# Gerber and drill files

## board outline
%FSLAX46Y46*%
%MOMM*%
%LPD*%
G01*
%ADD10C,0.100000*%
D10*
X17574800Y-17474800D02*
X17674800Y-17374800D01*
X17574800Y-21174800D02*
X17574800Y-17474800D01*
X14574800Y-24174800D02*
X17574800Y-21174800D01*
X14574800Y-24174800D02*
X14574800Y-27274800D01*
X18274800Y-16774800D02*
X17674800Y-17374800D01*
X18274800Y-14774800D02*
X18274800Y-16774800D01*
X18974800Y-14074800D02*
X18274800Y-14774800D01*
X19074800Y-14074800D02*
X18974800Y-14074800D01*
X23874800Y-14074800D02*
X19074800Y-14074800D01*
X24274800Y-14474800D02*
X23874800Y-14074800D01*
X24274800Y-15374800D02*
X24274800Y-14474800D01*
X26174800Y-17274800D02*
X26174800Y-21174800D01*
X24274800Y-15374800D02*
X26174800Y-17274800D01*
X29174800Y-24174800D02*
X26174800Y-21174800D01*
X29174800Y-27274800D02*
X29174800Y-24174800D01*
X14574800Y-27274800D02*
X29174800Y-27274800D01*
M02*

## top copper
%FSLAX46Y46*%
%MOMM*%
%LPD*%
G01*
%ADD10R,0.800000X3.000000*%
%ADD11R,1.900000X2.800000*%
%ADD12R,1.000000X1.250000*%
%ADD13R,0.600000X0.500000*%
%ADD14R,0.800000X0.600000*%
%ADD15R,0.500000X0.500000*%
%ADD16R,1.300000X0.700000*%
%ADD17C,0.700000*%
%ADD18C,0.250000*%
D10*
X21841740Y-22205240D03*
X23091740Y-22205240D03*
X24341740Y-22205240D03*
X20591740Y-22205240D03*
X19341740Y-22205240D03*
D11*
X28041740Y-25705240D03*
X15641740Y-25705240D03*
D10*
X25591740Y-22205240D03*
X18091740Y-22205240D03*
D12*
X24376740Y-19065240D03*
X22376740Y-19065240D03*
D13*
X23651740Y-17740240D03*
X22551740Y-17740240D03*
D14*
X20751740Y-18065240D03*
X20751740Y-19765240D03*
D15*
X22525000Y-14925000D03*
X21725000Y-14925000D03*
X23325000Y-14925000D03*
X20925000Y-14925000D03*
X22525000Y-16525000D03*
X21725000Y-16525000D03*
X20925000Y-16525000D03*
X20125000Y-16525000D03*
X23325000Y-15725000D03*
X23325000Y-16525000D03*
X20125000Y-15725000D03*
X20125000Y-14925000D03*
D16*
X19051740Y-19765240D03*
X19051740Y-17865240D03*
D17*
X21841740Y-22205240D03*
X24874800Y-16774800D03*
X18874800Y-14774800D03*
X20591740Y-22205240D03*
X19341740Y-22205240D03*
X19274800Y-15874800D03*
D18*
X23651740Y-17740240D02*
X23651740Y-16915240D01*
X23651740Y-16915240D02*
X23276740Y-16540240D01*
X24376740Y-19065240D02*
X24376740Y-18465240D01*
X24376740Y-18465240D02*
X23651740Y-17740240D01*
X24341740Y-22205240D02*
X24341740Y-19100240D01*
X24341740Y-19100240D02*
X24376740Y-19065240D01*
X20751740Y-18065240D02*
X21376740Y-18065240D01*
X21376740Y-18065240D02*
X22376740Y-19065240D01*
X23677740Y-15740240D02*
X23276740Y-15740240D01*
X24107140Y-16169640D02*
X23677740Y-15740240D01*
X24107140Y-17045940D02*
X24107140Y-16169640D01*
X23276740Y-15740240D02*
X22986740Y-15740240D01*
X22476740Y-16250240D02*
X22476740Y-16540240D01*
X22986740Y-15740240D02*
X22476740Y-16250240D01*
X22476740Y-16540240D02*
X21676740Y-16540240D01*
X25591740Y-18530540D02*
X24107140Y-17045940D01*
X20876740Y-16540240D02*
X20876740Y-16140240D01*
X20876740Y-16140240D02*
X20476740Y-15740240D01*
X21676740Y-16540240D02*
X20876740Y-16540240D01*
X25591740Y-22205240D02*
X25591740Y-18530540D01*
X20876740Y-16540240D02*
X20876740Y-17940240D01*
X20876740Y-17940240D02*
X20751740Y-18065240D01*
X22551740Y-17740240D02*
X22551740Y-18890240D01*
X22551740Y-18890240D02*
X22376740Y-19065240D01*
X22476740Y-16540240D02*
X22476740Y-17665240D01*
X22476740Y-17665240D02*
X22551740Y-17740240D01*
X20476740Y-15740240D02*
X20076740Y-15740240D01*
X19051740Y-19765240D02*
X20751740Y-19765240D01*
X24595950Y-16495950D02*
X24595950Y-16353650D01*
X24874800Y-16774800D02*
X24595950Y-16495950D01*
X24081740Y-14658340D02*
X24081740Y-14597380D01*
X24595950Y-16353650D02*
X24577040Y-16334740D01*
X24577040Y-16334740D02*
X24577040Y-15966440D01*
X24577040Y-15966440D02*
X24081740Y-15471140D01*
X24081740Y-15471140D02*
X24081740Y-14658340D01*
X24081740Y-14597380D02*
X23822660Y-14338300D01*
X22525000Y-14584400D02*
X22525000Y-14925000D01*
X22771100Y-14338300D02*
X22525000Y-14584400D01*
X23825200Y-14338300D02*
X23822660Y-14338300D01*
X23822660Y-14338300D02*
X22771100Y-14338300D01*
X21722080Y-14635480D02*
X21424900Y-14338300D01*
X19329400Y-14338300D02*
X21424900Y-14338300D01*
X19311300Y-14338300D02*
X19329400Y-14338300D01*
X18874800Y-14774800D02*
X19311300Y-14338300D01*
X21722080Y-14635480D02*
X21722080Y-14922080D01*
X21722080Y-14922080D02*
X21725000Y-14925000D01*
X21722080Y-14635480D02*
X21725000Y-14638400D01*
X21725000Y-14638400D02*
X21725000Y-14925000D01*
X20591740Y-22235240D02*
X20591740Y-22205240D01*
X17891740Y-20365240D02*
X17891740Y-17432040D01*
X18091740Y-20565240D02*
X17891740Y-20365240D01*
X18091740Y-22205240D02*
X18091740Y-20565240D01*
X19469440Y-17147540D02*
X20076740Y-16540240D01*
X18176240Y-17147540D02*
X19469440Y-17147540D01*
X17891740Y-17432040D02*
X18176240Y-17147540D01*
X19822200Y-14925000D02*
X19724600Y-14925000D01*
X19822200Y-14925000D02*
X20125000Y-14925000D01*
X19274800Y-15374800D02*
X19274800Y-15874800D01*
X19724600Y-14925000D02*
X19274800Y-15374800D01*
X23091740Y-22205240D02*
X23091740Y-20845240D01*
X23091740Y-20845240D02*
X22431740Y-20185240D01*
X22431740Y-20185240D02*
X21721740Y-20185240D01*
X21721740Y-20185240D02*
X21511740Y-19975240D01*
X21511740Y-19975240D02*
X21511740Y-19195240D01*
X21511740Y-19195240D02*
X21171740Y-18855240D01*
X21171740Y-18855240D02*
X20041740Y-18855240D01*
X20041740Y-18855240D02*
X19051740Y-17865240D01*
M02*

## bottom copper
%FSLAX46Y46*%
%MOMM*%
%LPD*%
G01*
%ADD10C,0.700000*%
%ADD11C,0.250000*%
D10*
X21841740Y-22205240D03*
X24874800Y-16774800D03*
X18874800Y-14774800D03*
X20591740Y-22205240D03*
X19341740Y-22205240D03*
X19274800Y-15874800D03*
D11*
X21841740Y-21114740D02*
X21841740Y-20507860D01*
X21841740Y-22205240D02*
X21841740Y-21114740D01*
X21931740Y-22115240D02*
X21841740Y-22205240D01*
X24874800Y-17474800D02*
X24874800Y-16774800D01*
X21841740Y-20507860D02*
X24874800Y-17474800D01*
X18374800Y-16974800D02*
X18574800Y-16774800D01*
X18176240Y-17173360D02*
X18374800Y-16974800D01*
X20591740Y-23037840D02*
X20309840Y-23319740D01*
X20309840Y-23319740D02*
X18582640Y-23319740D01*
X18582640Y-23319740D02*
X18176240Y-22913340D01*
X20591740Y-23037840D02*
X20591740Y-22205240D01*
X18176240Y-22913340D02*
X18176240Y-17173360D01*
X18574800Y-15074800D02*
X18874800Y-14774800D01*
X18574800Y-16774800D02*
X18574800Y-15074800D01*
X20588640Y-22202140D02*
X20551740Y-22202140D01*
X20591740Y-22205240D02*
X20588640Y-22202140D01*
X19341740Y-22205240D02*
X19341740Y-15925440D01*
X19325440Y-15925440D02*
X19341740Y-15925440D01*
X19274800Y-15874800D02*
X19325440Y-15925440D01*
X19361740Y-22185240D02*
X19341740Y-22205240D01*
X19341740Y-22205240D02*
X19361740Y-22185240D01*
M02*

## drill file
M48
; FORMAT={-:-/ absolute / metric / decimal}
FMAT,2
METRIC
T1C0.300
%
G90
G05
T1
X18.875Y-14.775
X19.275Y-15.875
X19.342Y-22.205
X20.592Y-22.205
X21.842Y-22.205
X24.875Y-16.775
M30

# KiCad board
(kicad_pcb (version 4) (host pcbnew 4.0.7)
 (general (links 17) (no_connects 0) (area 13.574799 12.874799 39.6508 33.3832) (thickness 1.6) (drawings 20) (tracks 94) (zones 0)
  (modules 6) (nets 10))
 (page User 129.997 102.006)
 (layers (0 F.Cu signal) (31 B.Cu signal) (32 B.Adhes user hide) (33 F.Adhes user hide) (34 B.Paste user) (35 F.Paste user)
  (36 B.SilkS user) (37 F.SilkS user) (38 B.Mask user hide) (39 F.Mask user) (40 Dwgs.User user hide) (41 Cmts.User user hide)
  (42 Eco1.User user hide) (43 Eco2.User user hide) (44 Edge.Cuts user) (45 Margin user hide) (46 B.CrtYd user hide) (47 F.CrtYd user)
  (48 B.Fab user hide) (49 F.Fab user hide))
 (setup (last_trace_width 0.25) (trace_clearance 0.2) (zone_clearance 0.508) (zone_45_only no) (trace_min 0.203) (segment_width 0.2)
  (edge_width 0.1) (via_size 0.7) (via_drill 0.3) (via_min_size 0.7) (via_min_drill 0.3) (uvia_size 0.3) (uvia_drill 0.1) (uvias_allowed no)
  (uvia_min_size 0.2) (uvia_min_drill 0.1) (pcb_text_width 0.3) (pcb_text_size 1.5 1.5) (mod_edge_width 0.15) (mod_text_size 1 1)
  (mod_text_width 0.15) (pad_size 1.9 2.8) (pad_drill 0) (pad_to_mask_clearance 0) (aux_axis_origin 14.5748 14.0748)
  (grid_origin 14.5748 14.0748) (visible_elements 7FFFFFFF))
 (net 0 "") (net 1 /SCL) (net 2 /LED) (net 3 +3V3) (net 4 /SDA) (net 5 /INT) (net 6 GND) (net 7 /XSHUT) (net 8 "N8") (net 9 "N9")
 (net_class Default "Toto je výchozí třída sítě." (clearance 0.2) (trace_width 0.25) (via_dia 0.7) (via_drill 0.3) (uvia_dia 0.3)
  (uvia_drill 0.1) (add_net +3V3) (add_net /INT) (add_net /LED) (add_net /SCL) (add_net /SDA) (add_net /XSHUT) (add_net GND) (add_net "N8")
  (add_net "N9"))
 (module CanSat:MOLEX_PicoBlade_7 (layer F.Cu) (at 21.84174 24.74524)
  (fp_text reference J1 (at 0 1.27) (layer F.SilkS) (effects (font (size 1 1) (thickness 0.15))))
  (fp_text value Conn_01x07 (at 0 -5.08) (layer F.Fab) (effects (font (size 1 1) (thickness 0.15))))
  (pad 4 smd rect (at 0 -2.54) (size 0.8 3) (layers F.Cu F.Paste F.Mask) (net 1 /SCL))
  (pad 5 smd rect (at 1.25 -2.54) (size 0.8 3) (layers F.Cu F.Paste F.Mask) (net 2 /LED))
  (pad 6 smd rect (at 2.5 -2.54) (size 0.8 3) (layers F.Cu F.Paste F.Mask) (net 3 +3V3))
  (pad 3 smd rect (at -1.25 -2.54) (size 0.8 3) (layers F.Cu F.Paste F.Mask) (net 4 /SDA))
  (pad 2 smd rect (at -2.5 -2.54) (size 0.8 3) (layers F.Cu F.Paste F.Mask) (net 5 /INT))
  (pad "" smd rect (at 6.2 0.96) (size 1.9 2.8) (layers F.Cu F.Paste F.Mask))
  (pad "" smd rect (at -6.2 0.96) (size 1.9 2.8) (layers F.Cu F.Paste F.Mask))
  (pad 7 smd rect (at 3.75 -2.54) (size 0.8 3) (layers F.Cu F.Paste F.Mask) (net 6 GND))
  (pad 1 smd rect (at -3.75 -2.54) (size 0.8 3) (layers F.Cu F.Paste F.Mask) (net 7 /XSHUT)))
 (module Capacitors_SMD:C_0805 (layer F.Cu) (at 23.37674 19.06524 180)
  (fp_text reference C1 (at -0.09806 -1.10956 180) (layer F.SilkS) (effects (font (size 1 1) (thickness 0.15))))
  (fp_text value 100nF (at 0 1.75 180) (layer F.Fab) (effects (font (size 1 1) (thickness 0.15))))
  (pad 1 smd rect (at -1 0 180) (size 1 1.25) (layers F.Cu F.Paste F.Mask) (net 3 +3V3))
  (pad 2 smd rect (at 1 0 180) (size 1 1.25) (layers F.Cu F.Paste F.Mask) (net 6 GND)))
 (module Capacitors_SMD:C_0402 (layer F.Cu) (at 23.10174 17.74024 180)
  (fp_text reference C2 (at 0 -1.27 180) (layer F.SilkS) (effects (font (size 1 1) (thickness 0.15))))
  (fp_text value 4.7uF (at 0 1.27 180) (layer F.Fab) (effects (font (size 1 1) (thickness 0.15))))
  (pad 1 smd rect (at -0.55 0 180) (size 0.6 0.5) (layers F.Cu F.Paste F.Mask) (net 3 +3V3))
  (pad 2 smd rect (at 0.55 0 180) (size 0.6 0.5) (layers F.Cu F.Paste F.Mask) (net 6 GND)))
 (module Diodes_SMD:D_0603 (layer F.Cu) (at 20.75174 18.91524 270)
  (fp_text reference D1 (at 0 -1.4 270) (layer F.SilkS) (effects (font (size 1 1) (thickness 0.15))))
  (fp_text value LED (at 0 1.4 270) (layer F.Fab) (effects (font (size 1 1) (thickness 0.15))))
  (pad 1 smd rect (at -0.85 0 270) (size 0.6 0.8) (layers F.Cu F.Paste F.Mask) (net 6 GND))
  (pad 2 smd rect (at 0.85 0 270) (size 0.6 0.8) (layers F.Cu F.Paste F.Mask) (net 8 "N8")))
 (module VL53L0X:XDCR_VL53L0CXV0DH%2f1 (layer F.Cu) (at 21.725 15.725 270)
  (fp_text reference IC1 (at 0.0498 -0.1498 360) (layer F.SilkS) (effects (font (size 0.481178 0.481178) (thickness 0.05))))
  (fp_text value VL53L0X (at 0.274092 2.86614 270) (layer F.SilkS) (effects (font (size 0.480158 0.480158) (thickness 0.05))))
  (pad 10 smd rect (at -0.8 -0.8 270) (size 0.5 0.5) (layers F.Cu F.Paste F.Mask) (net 1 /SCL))
  (pad 9 smd rect (at -0.8 0 270) (size 0.5 0.5) (layers F.Cu F.Paste F.Mask) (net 4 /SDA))
  (pad 11 smd rect (at -0.8 -1.6 270) (size 0.5 0.5) (layers F.Cu F.Paste F.Mask))
  (pad 8 smd rect (at -0.8 0.8 270) (size 0.5 0.5) (layers F.Cu F.Paste F.Mask) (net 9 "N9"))
  (pad 2 smd rect (at 0.8 -0.8 270) (size 0.5 0.5) (layers F.Cu F.Paste F.Mask) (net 6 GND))
  (pad 3 smd rect (at 0.8 0 270) (size 0.5 0.5) (layers F.Cu F.Paste F.Mask) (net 6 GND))
  (pad 4 smd rect (at 0.8 0.8 270) (size 0.5 0.5) (layers F.Cu F.Paste F.Mask) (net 6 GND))
  (pad 5 smd rect (at 0.8 1.6 270) (size 0.5 0.5) (layers F.Cu F.Paste F.Mask) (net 7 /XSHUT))
  (pad 12 smd rect (at 0 -1.6 270) (size 0.5 0.5) (layers F.Cu F.Paste F.Mask) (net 6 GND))
  (pad 1 smd rect (at 0.8 -1.6 270) (size 0.5 0.5) (layers F.Cu F.Paste F.Mask) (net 3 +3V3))
  (pad 6 smd rect (at 0 1.6 270) (size 0.5 0.5) (layers F.Cu F.Paste F.Mask) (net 6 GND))
  (pad 7 smd rect (at -0.8 1.6 270) (size 0.5 0.5) (layers F.Cu F.Paste F.Mask) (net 5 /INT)))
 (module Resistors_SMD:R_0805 (layer F.Cu) (at 19.05174 18.81524 90)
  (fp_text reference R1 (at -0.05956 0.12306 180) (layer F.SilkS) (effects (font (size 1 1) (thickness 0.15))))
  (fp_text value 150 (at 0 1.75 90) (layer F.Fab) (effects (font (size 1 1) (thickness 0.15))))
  (pad 1 smd rect (at -0.95 0 90) (size 0.7 1.3) (layers F.Cu F.Paste F.Mask) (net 8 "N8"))
  (pad 2 smd rect (at 0.95 0 90) (size 0.7 1.3) (layers F.Cu F.Paste F.Mask) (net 2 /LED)))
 (gr_line (start 17.5748 17.4748) (end 17.6748 17.3748) (angle 90) (layer Edge.Cuts) (width 0.1))
 (gr_line (start 17.5748 21.1748) (end 17.5748 17.4748) (angle 90) (layer Edge.Cuts) (width 0.1))
 (gr_line (start 14.5748 24.1748) (end 17.5748 21.1748) (angle 90) (layer Edge.Cuts) (width 0.1))
 (gr_line (start 14.5748 24.1748) (end 14.5748 27.2748) (angle 90) (layer Edge.Cuts) (width 0.1))
 (gr_line (start 18.2748 16.7748) (end 17.6748 17.3748) (angle 90) (layer Edge.Cuts) (width 0.1))
 (gr_line (start 18.2748 14.7748) (end 18.2748 16.7748) (angle 90) (layer Edge.Cuts) (width 0.1))
 (gr_line (start 18.9748 14.0748) (end 18.2748 14.7748) (angle 90) (layer Edge.Cuts) (width 0.1))
 (gr_line (start 19.0748 14.0748) (end 18.9748 14.0748) (angle 90) (layer Edge.Cuts) (width 0.1))
 (gr_line (start 23.8748 14.0748) (end 19.0748 14.0748) (angle 90) (layer Edge.Cuts) (width 0.1))
 (gr_line (start 24.2748 14.4748) (end 23.8748 14.0748) (angle 90) (layer Edge.Cuts) (width 0.1))
 (gr_line (start 24.2748 15.3748) (end 24.2748 14.4748) (angle 90) (layer Edge.Cuts) (width 0.1))
 (gr_line (start 26.1748 17.2748) (end 26.1748 21.1748) (angle 90) (layer Edge.Cuts) (width 0.1))
 (gr_line (start 24.2748 15.3748) (end 26.1748 17.2748) (angle 90) (layer Edge.Cuts) (width 0.1))
 (gr_line (start 29.1748 24.1748) (end 26.1748 21.1748) (angle 90) (layer Edge.Cuts) (width 0.1))
 (gr_line (start 29.1748 27.2748) (end 29.1748 24.1748) (angle 90) (layer Edge.Cuts) (width 0.1))
 (gr_line (start 14.5748 27.2748) (end 29.1748 27.2748) (angle 90) (layer Edge.Cuts) (width 0.1))
 (segment (start 23.65174 17.74024) (end 23.65174 16.91524) (width 0.25) (layer F.Cu) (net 3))
 (segment (start 23.65174 16.91524) (end 23.27674 16.54024) (width 0.25) (layer F.Cu) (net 3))
 (segment (start 24.37674 19.06524) (end 24.37674 18.46524) (width 0.25) (layer F.Cu) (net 3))
 (segment (start 24.37674 18.46524) (end 23.65174 17.74024) (width 0.25) (layer F.Cu) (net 3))
 (segment (start 24.34174 22.20524) (end 24.34174 19.10024) (width 0.25) (layer F.Cu) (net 3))
 (segment (start 24.34174 19.10024) (end 24.37674 19.06524) (width 0.25) (layer F.Cu) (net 3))
 (segment (start 20.75174 18.06524) (end 21.37674 18.06524) (width 0.25) (layer F.Cu) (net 6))
 (segment (start 21.37674 18.06524) (end 22.37674 19.06524) (width 0.25) (layer F.Cu) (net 6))
 (segment (start 23.67774 15.74024) (end 23.27674 15.74024) (width 0.25) (layer F.Cu) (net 6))
 (segment (start 24.10714 16.16964) (end 23.67774 15.74024) (width 0.25) (layer F.Cu) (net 6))
 (segment (start 24.10714 17.04594) (end 24.10714 16.16964) (width 0.25) (layer F.Cu) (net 6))
 (segment (start 23.27674 15.74024) (end 22.98674 15.74024) (width 0.25) (layer F.Cu) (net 6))
 (segment (start 22.47674 16.25024) (end 22.47674 16.54024) (width 0.25) (layer F.Cu) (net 6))
 (segment (start 22.98674 15.74024) (end 22.47674 16.25024) (width 0.25) (layer F.Cu) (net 6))
 (segment (start 22.47674 16.54024) (end 21.67674 16.54024) (width 0.25) (layer F.Cu) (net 6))
 (segment (start 25.59174 18.53054) (end 24.10714 17.04594) (width 0.25) (layer F.Cu) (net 6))
 (segment (start 20.87674 16.54024) (end 20.87674 16.14024) (width 0.25) (layer F.Cu) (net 6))
 (segment (start 20.87674 16.14024) (end 20.47674 15.74024) (width 0.25) (layer F.Cu) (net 6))
 (segment (start 21.67674 16.54024) (end 20.87674 16.54024) (width 0.25) (layer F.Cu) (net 6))
 (segment (start 25.59174 22.20524) (end 25.59174 18.53054) (width 0.25) (layer F.Cu) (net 6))
 (segment (start 20.87674 16.54024) (end 20.87674 17.94024) (width 0.25) (layer F.Cu) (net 6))
 (segment (start 20.87674 17.94024) (end 20.75174 18.06524) (width 0.25) (layer F.Cu) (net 6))
 (segment (start 22.55174 17.74024) (end 22.55174 18.89024) (width 0.25) (layer F.Cu) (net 6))
 (segment (start 22.55174 18.89024) (end 22.37674 19.06524) (width 0.25) (layer F.Cu) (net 6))
 (segment (start 22.47674 16.54024) (end 22.47674 17.66524) (width 0.25) (layer F.Cu) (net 6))
 (segment (start 22.47674 17.66524) (end 22.55174 17.74024) (width 0.25) (layer F.Cu) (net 6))
 (segment (start 20.47674 15.74024) (end 20.07674 15.74024) (width 0.25) (layer F.Cu) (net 6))
 (segment (start 19.05174 19.76524) (end 20.75174 19.76524) (width 0.25) (layer F.Cu) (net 8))
 (segment (start 21.84174 21.11474) (end 21.84174 20.50786) (width 0.25) (layer B.Cu) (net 1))
 (segment (start 21.84174 22.20524) (end 21.84174 21.11474) (width 0.25) (layer B.Cu) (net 1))
 (segment (start 21.93174 22.11524) (end 21.84174 22.20524) (width 0.25) (layer B.Cu) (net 1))
 (via (at 21.84174 22.20524) (size 0.7) (drill 0.3) (layers F.Cu B.Cu) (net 1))
 (segment (start 24.59595 16.49595) (end 24.59595 16.35365) (width 0.25) (layer F.Cu) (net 1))
 (segment (start 24.8748 16.7748) (end 24.59595 16.49595) (width 0.25) (layer F.Cu) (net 1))
 (via (at 24.8748 16.7748) (size 0.7) (drill 0.3) (layers F.Cu B.Cu) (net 1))
 (segment (start 24.8748 17.4748) (end 24.8748 16.7748) (width 0.25) (layer B.Cu) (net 1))
 (segment (start 21.84174 20.50786) (end 24.8748 17.4748) (width 0.25) (layer B.Cu) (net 1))
 (segment (start 24.08174 14.65834) (end 24.08174 14.59738) (width 0.25) (layer F.Cu) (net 1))
 (segment (start 24.59595 16.35365) (end 24.57704 16.33474) (width 0.25) (layer F.Cu) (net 1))
 (segment (start 24.57704 16.33474) (end 24.57704 15.96644) (width 0.25) (layer F.Cu) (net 1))
 (segment (start 24.57704 15.96644) (end 24.08174 15.47114) (width 0.25) (layer F.Cu) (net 1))
 (segment (start 24.08174 15.47114) (end 24.08174 14.65834) (width 0.25) (layer F.Cu) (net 1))
 (segment (start 24.08174 14.59738) (end 23.82266 14.3383) (width 0.25) (layer F.Cu) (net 1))
 (segment (start 22.525 14.5844) (end 22.525 14.925) (width 0.25) (layer F.Cu) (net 1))
 (segment (start 22.7711 14.3383) (end 22.525 14.5844) (width 0.25) (layer F.Cu) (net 1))
 (segment (start 23.8252 14.3383) (end 23.82266 14.3383) (width 0.25) (layer F.Cu) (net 1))
 (segment (start 23.82266 14.3383) (end 22.7711 14.3383) (width 0.25) (layer F.Cu) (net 1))
 (segment (start 18.3748 16.9748) (end 18.5748 16.7748) (width 0.25) (layer B.Cu) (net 4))
 (segment (start 21.72208 14.63548) (end 21.4249 14.3383) (width 0.25) (layer F.Cu) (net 4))
 (segment (start 19.3294 14.3383) (end 21.4249 14.3383) (width 0.25) (layer F.Cu) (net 4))
 (segment (start 18.17624 17.17336) (end 18.3748 16.9748) (width 0.25) (layer B.Cu) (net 4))
 (segment (start 20.59174 23.03784) (end 20.30984 23.31974) (width 0.25) (layer B.Cu) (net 4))
 (segment (start 20.30984 23.31974) (end 18.58264 23.31974) (width 0.25) (layer B.Cu) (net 4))
 (segment (start 18.58264 23.31974) (end 18.17624 22.91334) (width 0.25) (layer B.Cu) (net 4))
 (segment (start 20.59174 23.03784) (end 20.59174 22.20524) (width 0.25) (layer B.Cu) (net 4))
 (segment (start 18.17624 22.91334) (end 18.17624 17.17336) (width 0.25) (layer B.Cu) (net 4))
 (segment (start 19.3113 14.3383) (end 19.3294 14.3383) (width 0.25) (layer F.Cu) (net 4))
 (segment (start 18.8748 14.7748) (end 19.3113 14.3383) (width 0.25) (layer F.Cu) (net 4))
 (via (at 18.8748 14.7748) (size 0.7) (drill 0.3) (layers F.Cu B.Cu) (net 4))
 (segment (start 18.5748 15.0748) (end 18.8748 14.7748) (width 0.25) (layer B.Cu) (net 4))
 (segment (start 18.5748 16.7748) (end 18.5748 15.0748) (width 0.25) (layer B.Cu) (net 4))
 (segment (start 21.72208 14.63548) (end 21.72208 14.92208) (width 0.25) (layer F.Cu) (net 4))
 (segment (start 21.72208 14.92208) (end 21.725 14.925) (width 0.25) (layer F.Cu) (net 4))
 (segment (start 21.72208 14.63548) (end 21.725 14.6384) (width 0.25) (layer F.Cu) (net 4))
 (segment (start 21.725 14.6384) (end 21.725 14.925) (width 0.25) (layer F.Cu) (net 4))
 (via (at 20.59174 22.20524) (size 0.7) (drill 0.3) (layers F.Cu B.Cu) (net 4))
 (segment (start 20.59174 22.23524) (end 20.59174 22.20524) (width 0.25) (layer F.Cu) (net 4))
 (segment (start 20.58864 22.20214) (end 20.55174 22.20214) (width 0.25) (layer B.Cu) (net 4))
 (segment (start 20.59174 22.20524) (end 20.58864 22.20214) (width 0.25) (layer B.Cu) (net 4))
 (segment (start 17.89174 20.36524) (end 17.89174 17.43204) (width 0.25) (layer F.Cu) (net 7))
 (segment (start 18.09174 20.56524) (end 17.89174 20.36524) (width 0.25) (layer F.Cu) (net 7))
 (segment (start 18.09174 22.20524) (end 18.09174 20.56524) (width 0.25) (layer F.Cu) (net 7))
 (segment (start 19.46944 17.14754) (end 20.07674 16.54024) (width 0.25) (layer F.Cu) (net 7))
 (segment (start 18.17624 17.14754) (end 19.46944 17.14754) (width 0.25) (layer F.Cu) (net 7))
 (segment (start 17.89174 17.43204) (end 18.17624 17.14754) (width 0.25) (layer F.Cu) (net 7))
 (segment (start 19.8222 14.925) (end 19.7246 14.925) (width 0.25) (layer F.Cu) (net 5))
 (via (at 19.34174 22.20524) (size 0.7) (drill 0.3) (layers F.Cu B.Cu) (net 5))
 (segment (start 19.34174 22.20524) (end 19.34174 15.92544) (width 0.25) (layer B.Cu) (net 5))
 (segment (start 19.8222 14.925) (end 20.125 14.925) (width 0.25) (layer F.Cu) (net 5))
 (segment (start 19.32544 15.92544) (end 19.34174 15.92544) (width 0.25) (layer B.Cu) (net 5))
 (segment (start 19.2748 15.8748) (end 19.32544 15.92544) (width 0.25) (layer B.Cu) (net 5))
 (via (at 19.2748 15.8748) (size 0.7) (drill 0.3) (layers F.Cu B.Cu) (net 5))
 (segment (start 19.2748 15.3748) (end 19.2748 15.8748) (width 0.25) (layer F.Cu) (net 5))
 (segment (start 19.7246 14.925) (end 19.2748 15.3748) (width 0.25) (layer F.Cu) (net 5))
 (segment (start 19.36174 22.18524) (end 19.34174 22.20524) (width 0.25) (layer B.Cu) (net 5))
 (segment (start 19.34174 22.20524) (end 19.36174 22.18524) (width 0.25) (layer B.Cu) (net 5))
 (segment (start 23.09174 22.20524) (end 23.09174 20.84524) (width 0.25) (layer F.Cu) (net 2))
 (segment (start 23.09174 20.84524) (end 22.43174 20.18524) (width 0.25) (layer F.Cu) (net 2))
 (segment (start 22.43174 20.18524) (end 21.72174 20.18524) (width 0.25) (layer F.Cu) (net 2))
 (segment (start 21.72174 20.18524) (end 21.51174 19.97524) (width 0.25) (layer F.Cu) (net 2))
 (segment (start 21.51174 19.97524) (end 21.51174 19.19524) (width 0.25) (layer F.Cu) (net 2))
 (segment (start 21.51174 19.19524) (end 21.17174 18.85524) (width 0.25) (layer F.Cu) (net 2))
 (segment (start 21.17174 18.85524) (end 20.04174 18.85524) (width 0.25) (layer F.Cu) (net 2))
 (segment (start 20.04174 18.85524) (end 19.05174 17.86524) (width 0.25) (layer F.Cu) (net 2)))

